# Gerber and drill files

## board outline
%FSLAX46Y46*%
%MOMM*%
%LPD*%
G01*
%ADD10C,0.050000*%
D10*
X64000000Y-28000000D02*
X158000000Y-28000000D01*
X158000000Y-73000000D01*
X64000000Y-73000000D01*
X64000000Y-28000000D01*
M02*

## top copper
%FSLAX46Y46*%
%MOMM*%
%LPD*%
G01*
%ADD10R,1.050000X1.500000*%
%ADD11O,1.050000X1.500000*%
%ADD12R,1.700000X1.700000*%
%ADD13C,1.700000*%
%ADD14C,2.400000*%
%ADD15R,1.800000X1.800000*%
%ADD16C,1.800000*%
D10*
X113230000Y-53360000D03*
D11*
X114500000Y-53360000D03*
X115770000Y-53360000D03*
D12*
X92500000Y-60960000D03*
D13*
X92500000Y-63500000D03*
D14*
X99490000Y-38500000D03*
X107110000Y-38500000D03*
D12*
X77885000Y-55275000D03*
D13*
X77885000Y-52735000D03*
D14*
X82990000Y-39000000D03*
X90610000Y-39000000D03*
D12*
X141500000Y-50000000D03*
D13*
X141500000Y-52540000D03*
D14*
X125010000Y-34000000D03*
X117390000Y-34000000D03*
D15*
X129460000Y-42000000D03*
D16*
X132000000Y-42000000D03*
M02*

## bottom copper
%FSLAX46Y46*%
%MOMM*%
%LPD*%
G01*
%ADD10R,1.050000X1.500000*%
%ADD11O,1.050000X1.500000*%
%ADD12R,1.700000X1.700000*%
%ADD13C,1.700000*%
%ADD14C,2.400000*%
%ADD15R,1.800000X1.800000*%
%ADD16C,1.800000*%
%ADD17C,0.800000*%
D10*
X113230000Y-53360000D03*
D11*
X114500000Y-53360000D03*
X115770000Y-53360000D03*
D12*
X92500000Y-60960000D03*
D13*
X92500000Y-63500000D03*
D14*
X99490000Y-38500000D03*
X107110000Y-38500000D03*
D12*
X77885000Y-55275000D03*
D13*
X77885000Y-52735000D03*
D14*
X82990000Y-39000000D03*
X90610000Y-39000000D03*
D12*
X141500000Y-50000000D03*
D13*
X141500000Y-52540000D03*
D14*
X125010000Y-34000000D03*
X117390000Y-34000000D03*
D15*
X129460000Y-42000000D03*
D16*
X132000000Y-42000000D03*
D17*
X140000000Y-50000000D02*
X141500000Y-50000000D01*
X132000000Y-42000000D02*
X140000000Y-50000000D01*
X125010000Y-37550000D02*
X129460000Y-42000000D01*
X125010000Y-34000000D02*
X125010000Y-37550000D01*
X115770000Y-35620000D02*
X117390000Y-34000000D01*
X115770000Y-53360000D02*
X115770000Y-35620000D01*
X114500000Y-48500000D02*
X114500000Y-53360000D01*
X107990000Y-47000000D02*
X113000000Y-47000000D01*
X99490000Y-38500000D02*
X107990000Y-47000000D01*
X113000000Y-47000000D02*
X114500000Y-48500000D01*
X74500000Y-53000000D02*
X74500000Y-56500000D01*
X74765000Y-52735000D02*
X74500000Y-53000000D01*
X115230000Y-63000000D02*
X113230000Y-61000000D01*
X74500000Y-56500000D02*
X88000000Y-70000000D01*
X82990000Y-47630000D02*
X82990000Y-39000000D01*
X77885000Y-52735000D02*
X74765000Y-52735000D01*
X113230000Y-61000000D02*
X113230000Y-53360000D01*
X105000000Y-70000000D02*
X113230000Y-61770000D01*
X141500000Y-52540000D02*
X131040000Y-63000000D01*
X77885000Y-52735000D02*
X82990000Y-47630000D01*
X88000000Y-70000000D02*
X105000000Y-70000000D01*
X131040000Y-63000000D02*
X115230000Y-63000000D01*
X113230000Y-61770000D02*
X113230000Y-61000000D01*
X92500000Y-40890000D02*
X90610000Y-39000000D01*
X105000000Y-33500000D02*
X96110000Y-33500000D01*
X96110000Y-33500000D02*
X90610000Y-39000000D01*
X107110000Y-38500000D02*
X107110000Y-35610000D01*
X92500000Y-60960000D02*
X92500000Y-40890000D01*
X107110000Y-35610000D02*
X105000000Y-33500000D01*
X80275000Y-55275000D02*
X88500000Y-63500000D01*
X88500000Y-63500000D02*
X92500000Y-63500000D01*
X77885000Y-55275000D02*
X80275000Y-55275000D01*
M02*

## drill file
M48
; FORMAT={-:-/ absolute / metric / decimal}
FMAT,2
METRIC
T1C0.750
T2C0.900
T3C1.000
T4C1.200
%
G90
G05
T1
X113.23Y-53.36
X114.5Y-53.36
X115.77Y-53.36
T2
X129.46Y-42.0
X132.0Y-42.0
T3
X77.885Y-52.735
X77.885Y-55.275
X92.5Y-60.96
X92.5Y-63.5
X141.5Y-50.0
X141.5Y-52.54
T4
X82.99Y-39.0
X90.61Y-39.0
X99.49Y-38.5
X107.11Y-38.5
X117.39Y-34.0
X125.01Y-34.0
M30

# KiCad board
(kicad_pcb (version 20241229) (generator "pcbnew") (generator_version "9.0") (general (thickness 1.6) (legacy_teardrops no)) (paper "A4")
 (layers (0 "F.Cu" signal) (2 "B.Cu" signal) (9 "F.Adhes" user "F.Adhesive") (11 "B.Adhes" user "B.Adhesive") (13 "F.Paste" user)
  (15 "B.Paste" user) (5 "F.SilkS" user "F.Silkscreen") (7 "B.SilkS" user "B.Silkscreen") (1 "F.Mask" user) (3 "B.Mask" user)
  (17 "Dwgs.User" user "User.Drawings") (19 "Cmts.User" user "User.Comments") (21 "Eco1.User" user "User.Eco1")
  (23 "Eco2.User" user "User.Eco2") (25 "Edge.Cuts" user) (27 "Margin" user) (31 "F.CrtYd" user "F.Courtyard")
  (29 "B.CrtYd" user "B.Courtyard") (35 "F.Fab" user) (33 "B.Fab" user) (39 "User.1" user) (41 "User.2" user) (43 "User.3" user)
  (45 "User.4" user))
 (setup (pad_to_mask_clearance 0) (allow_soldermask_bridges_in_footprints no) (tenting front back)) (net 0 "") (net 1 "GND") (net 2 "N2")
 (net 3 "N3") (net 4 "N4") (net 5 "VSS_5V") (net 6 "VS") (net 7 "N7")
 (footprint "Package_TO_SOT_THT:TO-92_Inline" (layer "F.Cu") (at 113.23 53.36)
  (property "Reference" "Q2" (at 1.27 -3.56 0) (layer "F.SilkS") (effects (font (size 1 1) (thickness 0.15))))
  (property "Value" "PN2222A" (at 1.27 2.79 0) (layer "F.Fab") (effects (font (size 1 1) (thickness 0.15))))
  (pad "1" thru_hole rect (at 0 0) (size 1.05 1.5) (drill 0.75) (layers "*.Cu" "*.Mask") (remove_unused_layers no) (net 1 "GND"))
  (pad "2" thru_hole oval (at 1.27 0) (size 1.05 1.5) (drill 0.75) (layers "*.Cu" "*.Mask") (remove_unused_layers no) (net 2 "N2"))
  (pad "3" thru_hole oval (at 2.54 0) (size 1.05 1.5) (drill 0.75) (layers "*.Cu" "*.Mask") (remove_unused_layers no) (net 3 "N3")))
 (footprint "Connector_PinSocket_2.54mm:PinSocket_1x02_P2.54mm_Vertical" (layer "F.Cu") (at 92.5 60.96)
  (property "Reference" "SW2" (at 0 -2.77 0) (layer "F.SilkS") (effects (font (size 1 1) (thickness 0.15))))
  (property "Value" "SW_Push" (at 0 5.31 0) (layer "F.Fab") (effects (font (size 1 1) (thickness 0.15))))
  (pad "1" thru_hole rect (at 0 0) (size 1.7 1.7) (drill 1) (layers "*.Cu" "*.Mask") (remove_unused_layers no) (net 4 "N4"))
  (pad "2" thru_hole circle (at 0 2.54) (size 1.7 1.7) (drill 1) (layers "*.Cu" "*.Mask") (remove_unused_layers no) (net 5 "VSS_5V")))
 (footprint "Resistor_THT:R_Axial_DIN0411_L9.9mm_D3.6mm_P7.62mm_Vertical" (layer "F.Cu") (at 99.49 38.5)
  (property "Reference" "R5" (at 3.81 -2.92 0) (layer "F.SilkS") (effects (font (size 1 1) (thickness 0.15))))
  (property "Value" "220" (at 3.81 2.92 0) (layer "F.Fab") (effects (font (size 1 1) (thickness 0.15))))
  (pad "1" thru_hole circle (at 0 0) (size 2.4 2.4) (drill 1.2) (layers "*.Cu" "*.Mask") (remove_unused_layers no) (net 2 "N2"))
  (pad "2" thru_hole circle (at 7.62 0) (size 2.4 2.4) (drill 1.2) (layers "*.Cu" "*.Mask") (remove_unused_layers no) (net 4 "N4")))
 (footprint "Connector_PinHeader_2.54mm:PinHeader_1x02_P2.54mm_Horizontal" (layer "F.Cu") (at 77.885 55.275 180)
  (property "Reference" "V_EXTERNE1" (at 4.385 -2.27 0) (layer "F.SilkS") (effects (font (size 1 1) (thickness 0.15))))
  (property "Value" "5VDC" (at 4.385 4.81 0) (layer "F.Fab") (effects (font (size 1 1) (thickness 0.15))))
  (pad "1" thru_hole rect (at 0 0 180) (size 1.7 1.7) (drill 1) (layers "*.Cu" "*.Mask") (remove_unused_layers no) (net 5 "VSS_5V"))
  (pad "2" thru_hole circle (at 0 2.54 180) (size 1.7 1.7) (drill 1) (layers "*.Cu" "*.Mask") (remove_unused_layers no) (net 1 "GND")))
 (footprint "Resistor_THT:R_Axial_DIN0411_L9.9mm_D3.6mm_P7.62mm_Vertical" (layer "F.Cu") (at 82.99 39)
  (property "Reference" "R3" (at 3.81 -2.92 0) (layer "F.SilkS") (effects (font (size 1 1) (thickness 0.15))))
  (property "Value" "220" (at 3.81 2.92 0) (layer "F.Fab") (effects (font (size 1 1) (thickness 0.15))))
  (pad "1" thru_hole circle (at 0 0) (size 2.4 2.4) (drill 1.2) (layers "*.Cu" "*.Mask") (remove_unused_layers no) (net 1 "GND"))
  (pad "2" thru_hole circle (at 7.62 0) (size 2.4 2.4) (drill 1.2) (layers "*.Cu" "*.Mask") (remove_unused_layers no) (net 4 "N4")))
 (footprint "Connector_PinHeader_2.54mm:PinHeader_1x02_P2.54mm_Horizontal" (layer "F.Cu") (at 141.5 50)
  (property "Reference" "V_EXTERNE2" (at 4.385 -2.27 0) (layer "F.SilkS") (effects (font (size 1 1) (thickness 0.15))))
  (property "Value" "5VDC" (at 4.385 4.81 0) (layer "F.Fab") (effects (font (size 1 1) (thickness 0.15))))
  (pad "1" thru_hole rect (at 0 0) (size 1.7 1.7) (drill 1) (layers "*.Cu" "*.Mask") (remove_unused_layers no) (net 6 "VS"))
  (pad "2" thru_hole circle (at 0 2.54) (size 1.7 1.7) (drill 1) (layers "*.Cu" "*.Mask") (remove_unused_layers no) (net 1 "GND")))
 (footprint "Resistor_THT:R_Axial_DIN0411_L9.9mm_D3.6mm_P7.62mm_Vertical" (layer "F.Cu") (at 125.01 34 180)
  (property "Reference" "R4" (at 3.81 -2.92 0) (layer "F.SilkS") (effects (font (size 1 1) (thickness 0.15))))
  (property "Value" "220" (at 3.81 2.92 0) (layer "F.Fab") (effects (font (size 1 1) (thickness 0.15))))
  (pad "1" thru_hole circle (at 0 0 180) (size 2.4 2.4) (drill 1.2) (layers "*.Cu" "*.Mask") (remove_unused_layers no) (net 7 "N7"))
  (pad "2" thru_hole circle (at 7.62 0 180) (size 2.4 2.4) (drill 1.2) (layers "*.Cu" "*.Mask") (remove_unused_layers no) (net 3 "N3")))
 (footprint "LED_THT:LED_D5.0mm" (layer "F.Cu") (at 129.46 42)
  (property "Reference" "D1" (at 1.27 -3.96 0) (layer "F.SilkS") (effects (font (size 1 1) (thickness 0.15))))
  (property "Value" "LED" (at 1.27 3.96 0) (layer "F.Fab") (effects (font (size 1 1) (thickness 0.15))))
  (pad "1" thru_hole rect (at 0 0) (size 1.8 1.8) (drill 0.9) (layers "*.Cu" "*.Mask") (remove_unused_layers no) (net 7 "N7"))
  (pad "2" thru_hole circle (at 2.54 0) (size 1.8 1.8) (drill 0.9) (layers "*.Cu" "*.Mask") (remove_unused_layers no) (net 6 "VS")))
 (gr_rect (start 64 28) (end 158 73) (stroke (width 0.05) (type default)) (fill no) (layer "Edge.Cuts"))
 (segment (start 140 50) (end 141.5 50) (width 0.8) (layer "B.Cu") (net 6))
 (segment (start 132 42) (end 140 50) (width 0.8) (layer "B.Cu") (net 6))
 (segment (start 125.01 37.55) (end 129.46 42) (width 0.8) (layer "B.Cu") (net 7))
 (segment (start 125.01 34) (end 125.01 37.55) (width 0.8) (layer "B.Cu") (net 7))
 (segment (start 115.77 35.62) (end 117.39 34) (width 0.8) (layer "B.Cu") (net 3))
 (segment (start 115.77 53.36) (end 115.77 35.62) (width 0.8) (layer "B.Cu") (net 3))
 (segment (start 114.5 48.5) (end 114.5 53.36) (width 0.8) (layer "B.Cu") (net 2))
 (segment (start 107.99 47) (end 113 47) (width 0.8) (layer "B.Cu") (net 2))
 (segment (start 99.49 38.5) (end 107.99 47) (width 0.8) (layer "B.Cu") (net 2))
 (segment (start 113 47) (end 114.5 48.5) (width 0.8) (layer "B.Cu") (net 2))
 (segment (start 74.5 53) (end 74.5 56.5) (width 0.8) (layer "B.Cu") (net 1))
 (segment (start 74.765 52.735) (end 74.5 53) (width 0.8) (layer "B.Cu") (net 1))
 (segment (start 115.23 63) (end 113.23 61) (width 0.8) (layer "B.Cu") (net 1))
 (segment (start 74.5 56.5) (end 88 70) (width 0.8) (layer "B.Cu") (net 1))
 (segment (start 82.99 47.63) (end 82.99 39) (width 0.8) (layer "B.Cu") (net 1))
 (segment (start 77.885 52.735) (end 74.765 52.735) (width 0.8) (layer "B.Cu") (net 1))
 (segment (start 113.23 61) (end 113.23 53.36) (width 0.8) (layer "B.Cu") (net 1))
 (segment (start 105 70) (end 113.23 61.77) (width 0.8) (layer "B.Cu") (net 1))
 (segment (start 141.5 52.54) (end 131.04 63) (width 0.8) (layer "B.Cu") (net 1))
 (segment (start 77.885 52.735) (end 82.99 47.63) (width 0.8) (layer "B.Cu") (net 1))
 (segment (start 88 70) (end 105 70) (width 0.8) (layer "B.Cu") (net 1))
 (segment (start 131.04 63) (end 115.23 63) (width 0.8) (layer "B.Cu") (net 1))
 (segment (start 113.23 61.77) (end 113.23 61) (width 0.8) (layer "B.Cu") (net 1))
 (segment (start 92.5 40.89) (end 90.61 39) (width 0.8) (layer "B.Cu") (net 4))
 (segment (start 105 33.5) (end 96.11 33.5) (width 0.8) (layer "B.Cu") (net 4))
 (segment (start 96.11 33.5) (end 90.61 39) (width 0.8) (layer "B.Cu") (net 4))
 (segment (start 107.11 38.5) (end 107.11 35.61) (width 0.8) (layer "B.Cu") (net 4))
 (segment (start 92.5 60.96) (end 92.5 40.89) (width 0.8) (layer "B.Cu") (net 4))
 (segment (start 107.11 35.61) (end 105 33.5) (width 0.8) (layer "B.Cu") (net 4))
 (segment (start 80.275 55.275) (end 88.5 63.5) (width 0.8) (layer "B.Cu") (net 5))
 (segment (start 88.5 63.5) (end 92.5 63.5) (width 0.8) (layer "B.Cu") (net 5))
 (segment (start 77.885 55.275) (end 80.275 55.275) (width 0.8) (layer "B.Cu") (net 5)))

